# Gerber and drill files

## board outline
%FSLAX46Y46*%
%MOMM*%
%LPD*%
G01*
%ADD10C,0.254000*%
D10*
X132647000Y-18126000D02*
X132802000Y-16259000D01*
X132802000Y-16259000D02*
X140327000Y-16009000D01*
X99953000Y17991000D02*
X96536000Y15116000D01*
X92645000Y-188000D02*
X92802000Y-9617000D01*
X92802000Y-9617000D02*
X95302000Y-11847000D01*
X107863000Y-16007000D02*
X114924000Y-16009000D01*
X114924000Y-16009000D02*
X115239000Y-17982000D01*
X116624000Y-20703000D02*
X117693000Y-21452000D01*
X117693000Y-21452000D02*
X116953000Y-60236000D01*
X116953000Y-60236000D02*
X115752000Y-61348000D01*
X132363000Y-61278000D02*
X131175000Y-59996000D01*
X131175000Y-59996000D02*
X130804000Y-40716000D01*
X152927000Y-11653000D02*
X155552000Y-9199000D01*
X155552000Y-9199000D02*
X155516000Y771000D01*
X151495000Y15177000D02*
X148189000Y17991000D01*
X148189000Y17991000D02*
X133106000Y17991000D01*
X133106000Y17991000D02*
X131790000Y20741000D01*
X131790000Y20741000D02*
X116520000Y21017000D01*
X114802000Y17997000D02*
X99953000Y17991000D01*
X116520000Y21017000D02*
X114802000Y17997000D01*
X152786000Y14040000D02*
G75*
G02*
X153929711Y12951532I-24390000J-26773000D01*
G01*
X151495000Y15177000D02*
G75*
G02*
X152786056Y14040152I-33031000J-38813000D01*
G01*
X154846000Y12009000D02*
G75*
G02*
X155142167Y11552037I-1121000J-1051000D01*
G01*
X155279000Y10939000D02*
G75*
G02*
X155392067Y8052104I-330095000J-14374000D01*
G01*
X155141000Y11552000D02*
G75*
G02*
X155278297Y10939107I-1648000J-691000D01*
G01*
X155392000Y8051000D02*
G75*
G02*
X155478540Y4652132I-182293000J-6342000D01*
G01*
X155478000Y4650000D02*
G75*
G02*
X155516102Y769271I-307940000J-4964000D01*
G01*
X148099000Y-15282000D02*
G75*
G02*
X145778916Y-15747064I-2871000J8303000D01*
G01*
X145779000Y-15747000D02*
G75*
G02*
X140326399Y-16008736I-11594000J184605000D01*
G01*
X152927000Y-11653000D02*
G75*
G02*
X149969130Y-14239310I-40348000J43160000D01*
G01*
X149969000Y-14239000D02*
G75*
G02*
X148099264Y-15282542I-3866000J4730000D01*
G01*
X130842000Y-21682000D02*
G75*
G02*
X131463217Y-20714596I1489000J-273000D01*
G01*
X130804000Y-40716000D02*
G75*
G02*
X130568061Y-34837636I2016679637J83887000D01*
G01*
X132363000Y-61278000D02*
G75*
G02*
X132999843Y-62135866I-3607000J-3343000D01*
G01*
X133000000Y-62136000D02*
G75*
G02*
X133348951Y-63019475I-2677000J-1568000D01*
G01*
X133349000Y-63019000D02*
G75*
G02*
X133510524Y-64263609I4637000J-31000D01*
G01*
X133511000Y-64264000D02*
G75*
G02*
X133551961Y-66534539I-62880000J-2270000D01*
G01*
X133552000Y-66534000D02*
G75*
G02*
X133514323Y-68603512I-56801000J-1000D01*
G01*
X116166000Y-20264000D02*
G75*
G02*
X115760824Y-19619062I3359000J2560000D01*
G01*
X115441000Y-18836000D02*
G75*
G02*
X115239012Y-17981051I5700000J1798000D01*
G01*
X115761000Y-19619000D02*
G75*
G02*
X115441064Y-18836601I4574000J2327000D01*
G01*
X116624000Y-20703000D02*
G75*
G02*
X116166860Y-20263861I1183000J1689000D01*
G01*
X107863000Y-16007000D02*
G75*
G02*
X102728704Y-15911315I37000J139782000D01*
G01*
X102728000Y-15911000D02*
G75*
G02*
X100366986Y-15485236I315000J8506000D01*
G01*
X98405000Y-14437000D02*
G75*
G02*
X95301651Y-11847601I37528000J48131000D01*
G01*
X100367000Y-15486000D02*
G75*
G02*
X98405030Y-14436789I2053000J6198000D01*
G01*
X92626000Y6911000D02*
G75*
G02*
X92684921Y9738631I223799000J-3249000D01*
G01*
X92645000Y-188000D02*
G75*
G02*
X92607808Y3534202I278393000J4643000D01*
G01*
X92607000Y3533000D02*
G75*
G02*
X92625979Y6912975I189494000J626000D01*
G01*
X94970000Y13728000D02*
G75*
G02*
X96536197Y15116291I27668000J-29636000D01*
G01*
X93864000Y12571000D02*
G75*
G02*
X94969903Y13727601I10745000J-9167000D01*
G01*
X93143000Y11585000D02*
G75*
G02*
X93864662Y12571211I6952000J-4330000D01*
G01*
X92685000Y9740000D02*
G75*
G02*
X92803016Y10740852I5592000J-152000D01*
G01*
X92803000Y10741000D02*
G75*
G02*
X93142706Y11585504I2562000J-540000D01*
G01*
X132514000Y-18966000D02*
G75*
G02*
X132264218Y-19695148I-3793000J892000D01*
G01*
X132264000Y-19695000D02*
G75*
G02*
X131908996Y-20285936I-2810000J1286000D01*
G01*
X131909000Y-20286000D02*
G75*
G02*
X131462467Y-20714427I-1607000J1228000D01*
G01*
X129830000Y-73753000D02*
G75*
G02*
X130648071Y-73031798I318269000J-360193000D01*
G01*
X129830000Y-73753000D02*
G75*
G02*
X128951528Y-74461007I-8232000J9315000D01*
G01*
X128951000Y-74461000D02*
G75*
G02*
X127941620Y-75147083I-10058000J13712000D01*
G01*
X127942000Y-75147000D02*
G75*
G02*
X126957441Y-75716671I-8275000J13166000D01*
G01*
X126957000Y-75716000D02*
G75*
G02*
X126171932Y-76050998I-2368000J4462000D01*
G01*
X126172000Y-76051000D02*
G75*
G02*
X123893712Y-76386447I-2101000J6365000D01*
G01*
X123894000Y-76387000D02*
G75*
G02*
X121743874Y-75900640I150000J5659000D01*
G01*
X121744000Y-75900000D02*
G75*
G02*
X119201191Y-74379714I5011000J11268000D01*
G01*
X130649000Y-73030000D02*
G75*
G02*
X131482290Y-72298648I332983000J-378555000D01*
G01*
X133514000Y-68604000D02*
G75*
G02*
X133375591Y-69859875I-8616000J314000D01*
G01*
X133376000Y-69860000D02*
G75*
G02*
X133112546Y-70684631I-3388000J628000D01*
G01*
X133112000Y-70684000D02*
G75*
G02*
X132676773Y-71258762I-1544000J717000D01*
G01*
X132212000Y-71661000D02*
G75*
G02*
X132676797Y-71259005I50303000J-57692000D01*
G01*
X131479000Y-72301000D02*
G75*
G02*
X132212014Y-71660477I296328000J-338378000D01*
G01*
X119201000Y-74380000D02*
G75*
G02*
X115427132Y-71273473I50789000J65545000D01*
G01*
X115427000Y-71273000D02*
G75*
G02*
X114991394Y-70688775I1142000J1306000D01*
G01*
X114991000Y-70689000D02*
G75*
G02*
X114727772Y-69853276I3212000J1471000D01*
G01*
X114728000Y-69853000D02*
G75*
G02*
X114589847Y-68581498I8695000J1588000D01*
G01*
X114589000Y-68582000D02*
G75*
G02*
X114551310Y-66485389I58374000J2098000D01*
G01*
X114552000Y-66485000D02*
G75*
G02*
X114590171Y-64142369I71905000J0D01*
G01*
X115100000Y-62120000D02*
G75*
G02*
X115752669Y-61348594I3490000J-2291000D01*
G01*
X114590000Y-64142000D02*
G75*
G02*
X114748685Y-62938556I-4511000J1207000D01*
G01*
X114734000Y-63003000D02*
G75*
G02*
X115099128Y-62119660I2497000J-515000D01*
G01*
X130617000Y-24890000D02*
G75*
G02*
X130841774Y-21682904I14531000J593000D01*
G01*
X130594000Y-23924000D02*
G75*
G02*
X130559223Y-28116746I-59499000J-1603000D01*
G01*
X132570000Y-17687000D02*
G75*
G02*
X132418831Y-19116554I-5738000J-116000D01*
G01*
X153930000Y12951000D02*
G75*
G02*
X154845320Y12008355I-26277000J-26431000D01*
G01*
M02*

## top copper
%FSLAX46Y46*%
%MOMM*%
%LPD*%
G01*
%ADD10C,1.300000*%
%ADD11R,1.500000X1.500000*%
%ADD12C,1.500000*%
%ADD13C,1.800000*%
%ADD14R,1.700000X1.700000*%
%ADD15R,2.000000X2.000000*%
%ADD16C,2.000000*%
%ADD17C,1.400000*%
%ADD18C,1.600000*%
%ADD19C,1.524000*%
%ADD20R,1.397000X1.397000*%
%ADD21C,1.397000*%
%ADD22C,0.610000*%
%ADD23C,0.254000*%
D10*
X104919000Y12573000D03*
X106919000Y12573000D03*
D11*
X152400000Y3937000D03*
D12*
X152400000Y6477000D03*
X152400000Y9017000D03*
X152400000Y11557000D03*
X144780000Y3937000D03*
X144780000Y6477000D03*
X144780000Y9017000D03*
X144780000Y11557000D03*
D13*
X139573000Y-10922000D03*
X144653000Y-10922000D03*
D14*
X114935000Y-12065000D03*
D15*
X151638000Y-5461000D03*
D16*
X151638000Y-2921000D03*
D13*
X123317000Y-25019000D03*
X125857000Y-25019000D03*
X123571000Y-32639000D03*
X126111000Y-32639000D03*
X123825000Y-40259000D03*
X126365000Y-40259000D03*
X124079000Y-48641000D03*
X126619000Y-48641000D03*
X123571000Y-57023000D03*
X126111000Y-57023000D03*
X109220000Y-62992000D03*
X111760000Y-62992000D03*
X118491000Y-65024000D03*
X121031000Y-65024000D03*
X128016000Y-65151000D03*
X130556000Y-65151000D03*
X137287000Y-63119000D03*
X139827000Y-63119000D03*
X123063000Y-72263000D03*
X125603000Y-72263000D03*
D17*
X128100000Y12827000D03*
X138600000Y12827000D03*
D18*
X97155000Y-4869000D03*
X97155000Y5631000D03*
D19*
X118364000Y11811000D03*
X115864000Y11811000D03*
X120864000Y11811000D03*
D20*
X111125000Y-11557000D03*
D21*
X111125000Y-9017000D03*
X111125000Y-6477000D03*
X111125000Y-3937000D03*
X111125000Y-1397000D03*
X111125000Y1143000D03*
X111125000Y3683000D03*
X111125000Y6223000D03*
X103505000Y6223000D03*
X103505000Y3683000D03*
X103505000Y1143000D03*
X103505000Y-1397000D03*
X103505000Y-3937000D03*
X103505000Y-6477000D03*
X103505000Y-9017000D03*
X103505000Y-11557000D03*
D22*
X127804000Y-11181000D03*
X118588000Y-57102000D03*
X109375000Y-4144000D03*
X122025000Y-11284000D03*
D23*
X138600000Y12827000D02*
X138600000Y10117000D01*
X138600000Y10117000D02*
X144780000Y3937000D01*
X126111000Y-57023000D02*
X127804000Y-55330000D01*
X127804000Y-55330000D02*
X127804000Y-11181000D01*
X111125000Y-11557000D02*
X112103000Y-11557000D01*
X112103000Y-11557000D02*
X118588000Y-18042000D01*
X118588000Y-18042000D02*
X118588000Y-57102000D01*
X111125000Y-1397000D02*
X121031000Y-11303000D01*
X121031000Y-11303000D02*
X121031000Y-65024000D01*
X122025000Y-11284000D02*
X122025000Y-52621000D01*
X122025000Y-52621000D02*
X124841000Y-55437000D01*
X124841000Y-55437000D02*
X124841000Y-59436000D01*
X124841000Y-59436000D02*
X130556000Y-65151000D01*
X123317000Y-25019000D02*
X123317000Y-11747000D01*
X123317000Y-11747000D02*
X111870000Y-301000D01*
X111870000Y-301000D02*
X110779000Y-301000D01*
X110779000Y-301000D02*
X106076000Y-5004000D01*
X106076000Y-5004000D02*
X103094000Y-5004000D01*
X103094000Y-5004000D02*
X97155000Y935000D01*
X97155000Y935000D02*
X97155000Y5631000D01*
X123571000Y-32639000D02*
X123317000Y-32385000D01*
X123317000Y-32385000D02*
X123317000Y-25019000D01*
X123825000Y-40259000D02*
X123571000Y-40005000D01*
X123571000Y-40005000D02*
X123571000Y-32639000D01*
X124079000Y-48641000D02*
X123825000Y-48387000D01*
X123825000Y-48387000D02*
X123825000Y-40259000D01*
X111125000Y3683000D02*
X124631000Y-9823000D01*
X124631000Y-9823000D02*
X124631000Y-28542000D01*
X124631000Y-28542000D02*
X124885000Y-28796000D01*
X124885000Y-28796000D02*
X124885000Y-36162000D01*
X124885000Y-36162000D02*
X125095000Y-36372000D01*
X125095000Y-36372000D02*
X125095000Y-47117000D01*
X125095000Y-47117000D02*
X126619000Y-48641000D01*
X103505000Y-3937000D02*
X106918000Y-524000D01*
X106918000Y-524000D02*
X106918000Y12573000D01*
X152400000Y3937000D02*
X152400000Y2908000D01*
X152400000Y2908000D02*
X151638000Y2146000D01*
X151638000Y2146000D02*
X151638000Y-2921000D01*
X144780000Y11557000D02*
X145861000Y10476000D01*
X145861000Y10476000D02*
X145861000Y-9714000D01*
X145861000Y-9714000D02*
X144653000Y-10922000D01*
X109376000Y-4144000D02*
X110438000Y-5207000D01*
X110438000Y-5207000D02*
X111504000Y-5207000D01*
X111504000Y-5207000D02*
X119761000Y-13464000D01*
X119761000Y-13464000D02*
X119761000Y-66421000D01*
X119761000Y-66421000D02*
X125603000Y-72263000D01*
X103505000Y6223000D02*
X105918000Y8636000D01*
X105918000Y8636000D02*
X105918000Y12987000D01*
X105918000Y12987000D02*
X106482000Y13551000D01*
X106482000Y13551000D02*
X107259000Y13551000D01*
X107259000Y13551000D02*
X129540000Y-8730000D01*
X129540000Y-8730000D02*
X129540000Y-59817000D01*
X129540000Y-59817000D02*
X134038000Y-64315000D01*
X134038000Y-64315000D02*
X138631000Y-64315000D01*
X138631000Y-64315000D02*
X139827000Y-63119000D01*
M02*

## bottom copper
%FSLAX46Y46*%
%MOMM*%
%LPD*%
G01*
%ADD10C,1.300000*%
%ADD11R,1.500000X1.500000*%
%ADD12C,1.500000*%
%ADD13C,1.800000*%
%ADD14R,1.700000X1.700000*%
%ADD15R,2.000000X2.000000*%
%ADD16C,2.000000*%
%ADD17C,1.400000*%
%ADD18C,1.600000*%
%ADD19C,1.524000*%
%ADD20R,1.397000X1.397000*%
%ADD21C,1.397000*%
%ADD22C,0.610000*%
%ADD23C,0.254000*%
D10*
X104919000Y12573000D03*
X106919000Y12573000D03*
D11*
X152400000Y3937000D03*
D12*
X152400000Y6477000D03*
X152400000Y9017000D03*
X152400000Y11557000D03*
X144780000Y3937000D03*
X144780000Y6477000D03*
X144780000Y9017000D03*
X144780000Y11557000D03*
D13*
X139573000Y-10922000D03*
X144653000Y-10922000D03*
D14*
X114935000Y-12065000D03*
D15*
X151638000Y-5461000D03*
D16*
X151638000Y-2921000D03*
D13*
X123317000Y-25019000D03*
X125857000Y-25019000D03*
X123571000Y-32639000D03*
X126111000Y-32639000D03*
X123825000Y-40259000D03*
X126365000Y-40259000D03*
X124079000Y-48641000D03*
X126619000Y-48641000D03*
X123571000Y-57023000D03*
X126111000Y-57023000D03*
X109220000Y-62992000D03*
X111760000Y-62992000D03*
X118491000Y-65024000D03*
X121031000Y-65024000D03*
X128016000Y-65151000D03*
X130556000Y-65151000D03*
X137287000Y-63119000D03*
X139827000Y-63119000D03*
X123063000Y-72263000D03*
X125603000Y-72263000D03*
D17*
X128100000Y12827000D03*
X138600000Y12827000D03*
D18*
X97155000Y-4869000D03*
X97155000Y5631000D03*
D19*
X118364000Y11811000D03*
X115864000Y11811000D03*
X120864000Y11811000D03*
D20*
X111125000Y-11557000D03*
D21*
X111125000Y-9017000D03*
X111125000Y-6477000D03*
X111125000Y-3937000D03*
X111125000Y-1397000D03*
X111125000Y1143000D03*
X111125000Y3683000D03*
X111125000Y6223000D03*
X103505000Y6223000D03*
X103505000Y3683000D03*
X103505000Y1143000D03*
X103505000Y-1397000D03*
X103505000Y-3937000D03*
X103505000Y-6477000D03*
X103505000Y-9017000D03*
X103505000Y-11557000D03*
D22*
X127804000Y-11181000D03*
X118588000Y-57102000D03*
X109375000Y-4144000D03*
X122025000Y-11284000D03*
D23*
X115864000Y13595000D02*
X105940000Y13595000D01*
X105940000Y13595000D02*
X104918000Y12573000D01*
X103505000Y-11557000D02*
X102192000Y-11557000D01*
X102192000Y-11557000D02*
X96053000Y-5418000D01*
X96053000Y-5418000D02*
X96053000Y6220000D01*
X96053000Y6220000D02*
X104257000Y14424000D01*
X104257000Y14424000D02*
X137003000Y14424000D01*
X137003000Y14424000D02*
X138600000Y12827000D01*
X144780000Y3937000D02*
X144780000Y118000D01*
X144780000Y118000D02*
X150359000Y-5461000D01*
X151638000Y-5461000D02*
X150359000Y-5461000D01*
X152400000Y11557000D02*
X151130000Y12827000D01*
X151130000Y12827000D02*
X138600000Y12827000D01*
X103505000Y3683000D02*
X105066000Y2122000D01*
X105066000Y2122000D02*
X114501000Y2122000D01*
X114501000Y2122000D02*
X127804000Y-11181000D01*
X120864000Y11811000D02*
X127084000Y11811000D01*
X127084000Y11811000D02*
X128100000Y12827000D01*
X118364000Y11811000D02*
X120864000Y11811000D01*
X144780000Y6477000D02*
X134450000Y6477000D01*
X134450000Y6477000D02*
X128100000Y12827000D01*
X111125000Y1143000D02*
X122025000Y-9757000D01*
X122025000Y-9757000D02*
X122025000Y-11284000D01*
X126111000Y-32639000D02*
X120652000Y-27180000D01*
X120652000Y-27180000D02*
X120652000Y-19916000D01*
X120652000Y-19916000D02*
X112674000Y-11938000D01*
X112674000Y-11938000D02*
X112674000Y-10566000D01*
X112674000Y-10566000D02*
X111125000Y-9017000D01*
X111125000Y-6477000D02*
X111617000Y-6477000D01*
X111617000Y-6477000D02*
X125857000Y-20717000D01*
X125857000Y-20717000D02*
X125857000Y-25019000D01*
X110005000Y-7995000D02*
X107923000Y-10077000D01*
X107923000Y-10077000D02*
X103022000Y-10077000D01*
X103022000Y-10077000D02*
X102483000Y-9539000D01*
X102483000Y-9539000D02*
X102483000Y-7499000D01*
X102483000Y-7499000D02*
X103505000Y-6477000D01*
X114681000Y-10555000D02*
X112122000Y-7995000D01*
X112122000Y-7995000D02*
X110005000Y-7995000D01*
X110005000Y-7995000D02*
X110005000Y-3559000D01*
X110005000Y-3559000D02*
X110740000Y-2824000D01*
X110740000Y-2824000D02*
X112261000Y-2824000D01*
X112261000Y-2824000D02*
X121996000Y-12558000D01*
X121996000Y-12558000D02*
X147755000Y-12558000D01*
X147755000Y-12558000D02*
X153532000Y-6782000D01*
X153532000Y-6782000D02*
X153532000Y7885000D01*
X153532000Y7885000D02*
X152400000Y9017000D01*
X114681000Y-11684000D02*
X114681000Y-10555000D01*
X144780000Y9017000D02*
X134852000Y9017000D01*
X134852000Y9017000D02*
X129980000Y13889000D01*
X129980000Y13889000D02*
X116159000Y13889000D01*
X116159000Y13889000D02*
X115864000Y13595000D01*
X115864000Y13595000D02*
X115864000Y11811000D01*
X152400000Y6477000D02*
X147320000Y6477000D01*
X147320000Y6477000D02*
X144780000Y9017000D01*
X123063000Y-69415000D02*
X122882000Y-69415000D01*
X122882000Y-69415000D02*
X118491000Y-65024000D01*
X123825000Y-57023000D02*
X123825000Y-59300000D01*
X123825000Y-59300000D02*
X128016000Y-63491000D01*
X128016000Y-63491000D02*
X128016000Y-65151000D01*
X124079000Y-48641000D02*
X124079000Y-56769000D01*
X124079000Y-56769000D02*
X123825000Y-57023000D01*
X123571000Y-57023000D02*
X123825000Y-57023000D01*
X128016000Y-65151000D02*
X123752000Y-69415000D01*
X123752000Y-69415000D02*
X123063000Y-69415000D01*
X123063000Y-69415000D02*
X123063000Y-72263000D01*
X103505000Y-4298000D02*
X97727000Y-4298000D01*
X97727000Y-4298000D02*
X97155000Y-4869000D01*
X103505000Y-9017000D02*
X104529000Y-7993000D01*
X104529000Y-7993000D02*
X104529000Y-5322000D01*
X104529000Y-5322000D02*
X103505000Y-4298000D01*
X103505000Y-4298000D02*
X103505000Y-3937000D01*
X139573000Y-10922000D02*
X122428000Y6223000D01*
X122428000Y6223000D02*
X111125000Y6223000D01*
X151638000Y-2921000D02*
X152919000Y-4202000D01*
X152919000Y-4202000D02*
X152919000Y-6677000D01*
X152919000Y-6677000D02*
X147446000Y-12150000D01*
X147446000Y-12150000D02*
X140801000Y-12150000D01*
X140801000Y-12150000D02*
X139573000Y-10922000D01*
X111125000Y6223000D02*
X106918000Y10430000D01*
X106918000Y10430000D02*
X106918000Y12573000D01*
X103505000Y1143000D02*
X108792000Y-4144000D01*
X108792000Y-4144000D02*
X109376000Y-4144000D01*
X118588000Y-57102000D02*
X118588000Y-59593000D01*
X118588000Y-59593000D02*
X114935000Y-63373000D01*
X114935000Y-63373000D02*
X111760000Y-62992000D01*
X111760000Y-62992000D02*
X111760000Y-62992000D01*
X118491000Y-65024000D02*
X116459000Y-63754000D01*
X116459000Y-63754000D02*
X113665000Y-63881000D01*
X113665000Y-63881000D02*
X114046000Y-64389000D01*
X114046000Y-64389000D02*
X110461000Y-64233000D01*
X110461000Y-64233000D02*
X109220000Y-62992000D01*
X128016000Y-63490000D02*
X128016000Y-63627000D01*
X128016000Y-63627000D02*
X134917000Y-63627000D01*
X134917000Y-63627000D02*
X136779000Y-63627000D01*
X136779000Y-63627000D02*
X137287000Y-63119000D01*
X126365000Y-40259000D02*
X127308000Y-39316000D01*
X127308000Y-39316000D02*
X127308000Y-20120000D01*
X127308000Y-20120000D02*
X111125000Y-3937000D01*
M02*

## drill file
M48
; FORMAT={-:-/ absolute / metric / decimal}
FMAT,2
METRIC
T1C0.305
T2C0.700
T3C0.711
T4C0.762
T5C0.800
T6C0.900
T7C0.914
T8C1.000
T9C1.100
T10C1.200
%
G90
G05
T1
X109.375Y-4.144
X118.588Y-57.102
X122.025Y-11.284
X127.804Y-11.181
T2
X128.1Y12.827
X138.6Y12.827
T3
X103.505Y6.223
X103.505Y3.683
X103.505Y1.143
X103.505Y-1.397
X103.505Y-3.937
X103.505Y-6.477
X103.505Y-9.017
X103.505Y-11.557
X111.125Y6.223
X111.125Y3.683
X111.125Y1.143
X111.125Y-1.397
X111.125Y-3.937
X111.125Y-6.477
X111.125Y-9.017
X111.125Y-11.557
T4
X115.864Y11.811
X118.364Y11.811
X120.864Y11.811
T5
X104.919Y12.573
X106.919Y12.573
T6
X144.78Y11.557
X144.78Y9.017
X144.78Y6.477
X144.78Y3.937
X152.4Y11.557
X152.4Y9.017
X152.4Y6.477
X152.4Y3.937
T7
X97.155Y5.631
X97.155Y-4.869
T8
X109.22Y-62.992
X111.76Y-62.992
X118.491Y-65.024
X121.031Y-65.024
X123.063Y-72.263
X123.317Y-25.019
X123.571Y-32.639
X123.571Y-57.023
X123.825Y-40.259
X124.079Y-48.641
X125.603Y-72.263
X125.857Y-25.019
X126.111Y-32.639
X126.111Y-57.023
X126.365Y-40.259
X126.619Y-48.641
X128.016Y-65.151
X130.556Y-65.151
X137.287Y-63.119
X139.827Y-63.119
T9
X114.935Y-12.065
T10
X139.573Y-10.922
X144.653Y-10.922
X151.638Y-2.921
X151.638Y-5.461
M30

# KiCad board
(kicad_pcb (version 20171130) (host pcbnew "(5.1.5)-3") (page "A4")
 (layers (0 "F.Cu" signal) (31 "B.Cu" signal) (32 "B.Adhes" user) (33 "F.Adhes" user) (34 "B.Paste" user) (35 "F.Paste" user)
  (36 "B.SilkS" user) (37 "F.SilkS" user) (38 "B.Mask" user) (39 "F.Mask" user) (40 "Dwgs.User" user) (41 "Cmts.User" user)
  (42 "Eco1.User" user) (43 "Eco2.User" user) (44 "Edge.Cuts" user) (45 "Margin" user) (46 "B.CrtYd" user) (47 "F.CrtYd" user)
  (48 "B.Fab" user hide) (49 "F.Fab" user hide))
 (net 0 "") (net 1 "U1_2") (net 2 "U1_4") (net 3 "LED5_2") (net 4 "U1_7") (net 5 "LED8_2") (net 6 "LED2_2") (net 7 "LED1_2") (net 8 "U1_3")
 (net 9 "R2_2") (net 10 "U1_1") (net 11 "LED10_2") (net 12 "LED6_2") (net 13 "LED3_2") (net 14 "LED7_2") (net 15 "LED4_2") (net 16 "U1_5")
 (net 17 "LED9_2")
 (segment (start 115.864 -13.595) (end 105.94 -13.595) (width 0.254) (layer "B.Cu") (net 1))
 (segment (start 105.94 -13.595) (end 104.918 -12.573) (width 0.254) (layer "B.Cu") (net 1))
 (segment (start 103.505 11.557) (end 102.192 11.557) (width 0.254) (layer "B.Cu") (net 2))
 (segment (start 102.192 11.557) (end 96.053 5.418) (width 0.254) (layer "B.Cu") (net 2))
 (segment (start 96.053 5.418) (end 96.053 -6.22) (width 0.254) (layer "B.Cu") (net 2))
 (segment (start 96.053 -6.22) (end 104.257 -14.424) (width 0.254) (layer "B.Cu") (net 2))
 (segment (start 104.257 -14.424) (end 137.003 -14.424) (width 0.254) (layer "B.Cu") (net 2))
 (segment (start 137.003 -14.424) (end 138.6 -12.827) (width 0.254) (layer "B.Cu") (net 2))
 (segment (start 144.78 -3.937) (end 144.78 -0.118) (width 0.254) (layer "B.Cu") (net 2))
 (segment (start 144.78 -0.118) (end 150.359 5.461) (width 0.254) (layer "B.Cu") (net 2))
 (segment (start 151.638 5.461) (end 150.359 5.461) (width 0.254) (layer "B.Cu") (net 2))
 (segment (start 152.4 -11.557) (end 151.13 -12.827) (width 0.254) (layer "B.Cu") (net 2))
 (segment (start 151.13 -12.827) (end 138.6 -12.827) (width 0.254) (layer "B.Cu") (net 2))
 (segment (start 103.505 -3.683) (end 105.066 -2.122) (width 0.254) (layer "B.Cu") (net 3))
 (segment (start 105.066 -2.122) (end 114.501 -2.122) (width 0.254) (layer "B.Cu") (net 3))
 (segment (start 114.501 -2.122) (end 127.804 11.181) (width 0.254) (layer "B.Cu") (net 3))
 (segment (start 120.864 -11.811) (end 127.084 -11.811) (width 0.254) (layer "B.Cu") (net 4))
 (segment (start 127.084 -11.811) (end 128.1 -12.827) (width 0.254) (layer "B.Cu") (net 4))
 (segment (start 118.364 -11.811) (end 120.864 -11.811) (width 0.254) (layer "B.Cu") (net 4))
 (segment (start 144.78 -6.477) (end 134.45 -6.477) (width 0.254) (layer "B.Cu") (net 4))
 (segment (start 134.45 -6.477) (end 128.1 -12.827) (width 0.254) (layer "B.Cu") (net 4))
 (segment (start 111.125 -1.143) (end 122.025 9.757) (width 0.254) (layer "B.Cu") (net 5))
 (segment (start 122.025 9.757) (end 122.025 11.284) (width 0.254) (layer "B.Cu") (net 5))
 (segment (start 126.111 32.639) (end 120.652 27.18) (width 0.254) (layer "B.Cu") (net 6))
 (segment (start 120.652 27.18) (end 120.652 19.916) (width 0.254) (layer "B.Cu") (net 6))
 (segment (start 120.652 19.916) (end 112.674 11.938) (width 0.254) (layer "B.Cu") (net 6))
 (segment (start 112.674 11.938) (end 112.674 10.566) (width 0.254) (layer "B.Cu") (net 6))
 (segment (start 112.674 10.566) (end 111.125 9.017) (width 0.254) (layer "B.Cu") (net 6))
 (segment (start 111.125 6.477) (end 111.617 6.477) (width 0.254) (layer "B.Cu") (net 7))
 (segment (start 111.617 6.477) (end 125.857 20.717) (width 0.254) (layer "B.Cu") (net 7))
 (segment (start 125.857 20.717) (end 125.857 25.019) (width 0.254) (layer "B.Cu") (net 7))
 (segment (start 110.005 7.995) (end 107.923 10.077) (width 0.254) (layer "B.Cu") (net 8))
 (segment (start 107.923 10.077) (end 103.022 10.077) (width 0.254) (layer "B.Cu") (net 8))
 (segment (start 103.022 10.077) (end 102.483 9.539) (width 0.254) (layer "B.Cu") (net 8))
 (segment (start 102.483 9.539) (end 102.483 7.499) (width 0.254) (layer "B.Cu") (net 8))
 (segment (start 102.483 7.499) (end 103.505 6.477) (width 0.254) (layer "B.Cu") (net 8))
 (segment (start 114.681 10.555) (end 112.122 7.995) (width 0.254) (layer "B.Cu") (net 8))
 (segment (start 112.122 7.995) (end 110.005 7.995) (width 0.254) (layer "B.Cu") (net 8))
 (segment (start 110.005 7.995) (end 110.005 3.559) (width 0.254) (layer "B.Cu") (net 8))
 (segment (start 110.005 3.559) (end 110.74 2.824) (width 0.254) (layer "B.Cu") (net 8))
 (segment (start 110.74 2.824) (end 112.261 2.824) (width 0.254) (layer "B.Cu") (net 8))
 (segment (start 112.261 2.824) (end 121.996 12.558) (width 0.254) (layer "B.Cu") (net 8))
 (segment (start 121.996 12.558) (end 147.755 12.558) (width 0.254) (layer "B.Cu") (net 8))
 (segment (start 147.755 12.558) (end 153.532 6.782) (width 0.254) (layer "B.Cu") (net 8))
 (segment (start 153.532 6.782) (end 153.532 -7.885) (width 0.254) (layer "B.Cu") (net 8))
 (segment (start 153.532 -7.885) (end 152.4 -9.017) (width 0.254) (layer "B.Cu") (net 8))
 (segment (start 114.681 11.684) (end 114.681 10.555) (width 0.254) (layer "B.Cu") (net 8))
 (segment (start 144.78 -9.017) (end 134.852 -9.017) (width 0.254) (layer "B.Cu") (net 1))
 (segment (start 134.852 -9.017) (end 129.98 -13.889) (width 0.254) (layer "B.Cu") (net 1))
 (segment (start 129.98 -13.889) (end 116.159 -13.889) (width 0.254) (layer "B.Cu") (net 1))
 (segment (start 116.159 -13.889) (end 115.864 -13.595) (width 0.254) (layer "B.Cu") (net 1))
 (segment (start 115.864 -13.595) (end 115.864 -11.811) (width 0.254) (layer "B.Cu") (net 1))
 (segment (start 152.4 -6.477) (end 147.32 -6.477) (width 0.254) (layer "B.Cu") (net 1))
 (segment (start 147.32 -6.477) (end 144.78 -9.017) (width 0.254) (layer "B.Cu") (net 1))
 (segment (start 123.063 69.415) (end 122.882 69.415) (width 0.254) (layer "B.Cu") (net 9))
 (segment (start 122.882 69.415) (end 118.491 65.024) (width 0.254) (layer "B.Cu") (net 9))
 (segment (start 123.825 57.023) (end 123.825 59.3) (width 0.254) (layer "B.Cu") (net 9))
 (segment (start 123.825 59.3) (end 128.016 63.491) (width 0.254) (layer "B.Cu") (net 9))
 (segment (start 128.016 63.491) (end 128.016 65.151) (width 0.254) (layer "B.Cu") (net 9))
 (segment (start 124.079 48.641) (end 124.079 56.769) (width 0.254) (layer "B.Cu") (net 9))
 (segment (start 124.079 56.769) (end 123.825 57.023) (width 0.254) (layer "B.Cu") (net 9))
 (segment (start 123.571 57.023) (end 123.825 57.023) (width 0.254) (layer "B.Cu") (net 9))
 (segment (start 128.016 65.151) (end 123.752 69.415) (width 0.254) (layer "B.Cu") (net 9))
 (segment (start 123.752 69.415) (end 123.063 69.415) (width 0.254) (layer "B.Cu") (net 9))
 (segment (start 123.063 69.415) (end 123.063 72.263) (width 0.254) (layer "B.Cu") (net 9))
 (segment (start 103.505 4.298) (end 97.727 4.298) (width 0.254) (layer "B.Cu") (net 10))
 (segment (start 97.727 4.298) (end 97.155 4.869) (width 0.254) (layer "B.Cu") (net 10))
 (segment (start 103.505 9.017) (end 104.529 7.993) (width 0.254) (layer "B.Cu") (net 10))
 (segment (start 104.529 7.993) (end 104.529 5.322) (width 0.254) (layer "B.Cu") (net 10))
 (segment (start 104.529 5.322) (end 103.505 4.298) (width 0.254) (layer "B.Cu") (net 10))
 (segment (start 103.505 4.298) (end 103.505 3.937) (width 0.254) (layer "B.Cu") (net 10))
 (segment (start 139.573 10.922) (end 122.428 -6.223) (width 0.254) (layer "B.Cu") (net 10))
 (segment (start 122.428 -6.223) (end 111.125 -6.223) (width 0.254) (layer "B.Cu") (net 10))
 (segment (start 151.638 2.921) (end 152.919 4.202) (width 0.254) (layer "B.Cu") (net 10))
 (segment (start 152.919 4.202) (end 152.919 6.677) (width 0.254) (layer "B.Cu") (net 10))
 (segment (start 152.919 6.677) (end 147.446 12.15) (width 0.254) (layer "B.Cu") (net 10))
 (segment (start 147.446 12.15) (end 140.801 12.15) (width 0.254) (layer "B.Cu") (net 10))
 (segment (start 140.801 12.15) (end 139.573 10.922) (width 0.254) (layer "B.Cu") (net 10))
 (segment (start 111.125 -6.223) (end 106.918 -10.43) (width 0.254) (layer "B.Cu") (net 10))
 (segment (start 106.918 -10.43) (end 106.918 -12.573) (width 0.254) (layer "B.Cu") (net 10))
 (segment (start 103.505 -1.143) (end 108.792 4.144) (width 0.254) (layer "B.Cu") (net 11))
 (segment (start 108.792 4.144) (end 109.376 4.144) (width 0.254) (layer "B.Cu") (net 11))
 (segment (start 118.588 57.102) (end 118.588 59.593) (width 0.254) (layer "B.Cu") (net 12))
 (segment (start 118.588 59.593) (end 114.935 63.373) (width 0.254) (layer "B.Cu") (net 12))
 (segment (start 114.935 63.373) (end 111.76 62.992) (width 0.254) (layer "B.Cu") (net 12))
 (segment (start 111.76 62.992) (end 111.76 62.992) (width 0.254) (layer "B.Cu") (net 12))
 (segment (start 118.491 65.024) (end 116.459 63.754) (width 0.254) (layer "B.Cu") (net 9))
 (segment (start 116.459 63.754) (end 113.665 63.881) (width 0.254) (layer "B.Cu") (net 9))
 (segment (start 113.665 63.881) (end 114.046 64.389) (width 0.254) (layer "B.Cu") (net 9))
 (segment (start 114.046 64.389) (end 110.461 64.233) (width 0.254) (layer "B.Cu") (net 9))
 (segment (start 110.461 64.233) (end 109.22 62.992) (width 0.254) (layer "B.Cu") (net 9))
 (segment (start 128.016 63.49) (end 128.016 63.627) (width 0.254) (layer "B.Cu") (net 9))
 (segment (start 128.016 63.627) (end 134.917 63.627) (width 0.254) (layer "B.Cu") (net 9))
 (segment (start 134.917 63.627) (end 136.779 63.627) (width 0.254) (layer "B.Cu") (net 9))
 (segment (start 136.779 63.627) (end 137.287 63.119) (width 0.254) (layer "B.Cu") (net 9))
 (segment (start 126.365 40.259) (end 127.308 39.316) (width 0.254) (layer "B.Cu") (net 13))
 (segment (start 127.308 39.316) (end 127.308 20.12) (width 0.254) (layer "B.Cu") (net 13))
 (segment (start 127.308 20.12) (end 111.125 3.937) (width 0.254) (layer "B.Cu") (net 13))
 (gr_line (start 132.647 18.126) (end 132.802 16.259) (width 0.254) (layer "Edge.Cuts"))
 (gr_line (start 132.802 16.259) (end 140.327 16.009) (width 0.254) (layer "Edge.Cuts"))
 (gr_line (start 99.953 -17.991) (end 96.536 -15.116) (width 0.254) (layer "Edge.Cuts"))
 (gr_line (start 92.645 0.188) (end 92.802 9.617) (width 0.254) (layer "Edge.Cuts"))
 (gr_line (start 92.802 9.617) (end 95.302 11.847) (width 0.254) (layer "Edge.Cuts"))
 (gr_line (start 107.863 16.007) (end 114.924 16.009) (width 0.254) (layer "Edge.Cuts"))
 (gr_line (start 114.924 16.009) (end 115.239 17.982) (width 0.254) (layer "Edge.Cuts"))
 (gr_line (start 116.624 20.703) (end 117.693 21.452) (width 0.254) (layer "Edge.Cuts"))
 (gr_line (start 117.693 21.452) (end 116.953 60.236) (width 0.254) (layer "Edge.Cuts"))
 (gr_line (start 116.953 60.236) (end 115.752 61.348) (width 0.254) (layer "Edge.Cuts"))
 (gr_line (start 132.363 61.278) (end 131.175 59.996) (width 0.254) (layer "Edge.Cuts"))
 (gr_line (start 131.175 59.996) (end 130.804 40.716) (width 0.254) (layer "Edge.Cuts"))
 (gr_line (start 152.927 11.653) (end 155.552 9.199) (width 0.254) (layer "Edge.Cuts"))
 (gr_line (start 155.552 9.199) (end 155.516 -0.771) (width 0.254) (layer "Edge.Cuts"))
 (gr_line (start 151.495 -15.177) (end 148.189 -17.991) (width 0.254) (layer "Edge.Cuts"))
 (gr_line (start 148.189 -17.991) (end 133.106 -17.991) (width 0.254) (layer "Edge.Cuts"))
 (gr_line (start 133.106 -17.991) (end 131.79 -20.741) (width 0.254) (layer "Edge.Cuts"))
 (gr_line (start 131.79 -20.741) (end 116.52 -21.017) (width 0.254) (layer "Edge.Cuts"))
 (gr_line (start 114.802 -17.997) (end 99.953 -17.991) (width 0.254) (layer "Edge.Cuts"))
 (gr_line (start 116.52 -21.017) (end 114.802 -17.997) (width 0.254) (layer "Edge.Cuts"))
 (gr_arc (start 128.396 12.733) (end 152.786 -14.04) (angle 2.498) (width 0.254) (layer "Edge.Cuts"))
 (gr_arc (start 118.464 23.636) (end 151.495 -15.177) (angle 1.934) (width 0.254) (layer "Edge.Cuts"))
 (gr_arc (start 153.725 -10.958) (end 154.846 -12.009) (angle 20.412) (width 0.254) (layer "Edge.Cuts"))
 (gr_arc (start -174.816 3.435) (end 155.279 -10.939) (angle 0.501) (width 0.254) (layer "Edge.Cuts"))
 (gr_arc (start 153.493 -10.861) (end 155.141 -11.552) (angle 20.243) (width 0.254) (layer "Edge.Cuts"))
 (gr_arc (start -26.901 -1.709) (end 155.392 -8.051) (angle 1.068) (width 0.254) (layer "Edge.Cuts"))
 (gr_arc (start -152.462 0.314) (end 155.478 -4.65) (angle 0.722) (width 0.254) (layer "Edge.Cuts"))
 (gr_arc (start 145.228 6.979) (end 148.099 15.282) (angle 15.479) (width 0.254) (layer "Edge.Cuts"))
 (gr_arc (start 134.185 -168.858) (end 145.779 15.747) (angle 1.691) (width 0.254) (layer "Edge.Cuts"))
 (gr_arc (start 112.579 -31.507) (end 152.927 11.653) (angle 3.811) (width 0.254) (layer "Edge.Cuts"))
 (gr_arc (start 146.103 9.509) (end 149.969 14.239) (angle 20.187) (width 0.254) (layer "Edge.Cuts"))
 (gr_arc (start 132.331 21.955) (end 130.842 21.682) (angle 44.634) (width 0.254) (layer "Edge.Cuts"))
 (gr_arc (start 4493.463 -43.171) (end 130.804 40.716) (angle 0.167) (width 0.254) (layer "Edge.Cuts"))
 (gr_arc (start 128.756 64.621) (end 132.363 61.278) (angle 12.472) (width 0.254) (layer "Edge.Cuts"))
 (gr_arc (start 130.323 63.704) (end 133 62.136) (angle 17.612) (width 0.254) (layer "Edge.Cuts"))
 (gr_arc (start 137.986 63.05) (end 133.349 63.019) (angle 344.445) (width 0.254) (layer "Edge.Cuts"))
 (gr_arc (start 70.631 66.534) (end 133.511 64.264) (angle 2.068) (width 0.254) (layer "Edge.Cuts"))
 (gr_arc (start 76.751 66.535) (end 133.552 66.534) (angle 2.088) (width 0.254) (layer "Edge.Cuts"))
 (gr_arc (start 119.525 17.704) (end 116.166 20.264) (angle 10.347) (width 0.254) (layer "Edge.Cuts"))
 (gr_arc (start 121.141 17.038) (end 115.441 18.836) (angle 8.429) (width 0.254) (layer "Edge.Cuts"))
 (gr_arc (start 120.335 17.292) (end 115.761 19.619) (angle 9.448) (width 0.254) (layer "Edge.Cuts"))
 (gr_arc (start 117.807 19.014) (end 116.624 20.703) (angle 17.683) (width 0.254) (layer "Edge.Cuts"))
 (gr_arc (start 107.9 -123.775) (end 107.863 16.007) (angle 2.105) (width 0.254) (layer "Edge.Cuts"))
 (gr_arc (start 103.043 7.405) (end 102.728 15.911) (angle 16.203) (width 0.254) (layer "Edge.Cuts"))
 (gr_arc (start 135.933 -33.694) (end 98.405 14.437) (angle 3.795) (width 0.254) (layer "Edge.Cuts"))
 (gr_arc (start 102.42 9.288) (end 100.367 15.486) (angle 19.62) (width 0.254) (layer "Edge.Cuts"))
 (gr_arc (start 316.425 -3.662) (end 92.626 -6.911) (angle 0.724) (width 0.254) (layer "Edge.Cuts"))
 (gr_arc (start 371.038 -4.455) (end 92.645 0.188) (angle 0.766) (width 0.254) (layer "Edge.Cuts"))
 (gr_arc (start 282.101 -4.159) (end 92.607 -3.533) (angle 1.022) (width 0.254) (layer "Edge.Cuts"))
 (gr_arc (start 122.638 15.908) (end 94.97 -13.728) (angle 2.958) (width 0.254) (layer "Edge.Cuts"))
 (gr_arc (start 104.609 -3.404) (end 93.864 -12.571) (angle 6.495) (width 0.254) (layer "Edge.Cuts"))
 (gr_arc (start 100.095 -7.255) (end 93.143 -11.585) (angle 8.557) (width 0.254) (layer "Edge.Cuts"))
 (gr_arc (start 98.277 -9.588) (end 92.685 -9.74) (angle 10.336) (width 0.254) (layer "Edge.Cuts"))
 (gr_arc (start 95.365 -10.201) (end 92.803 -10.741) (angle 20.021) (width 0.254) (layer "Edge.Cuts"))
 (gr_arc (start 128.721 18.074) (end 132.514 18.966) (angle 11.352) (width 0.254) (layer "Edge.Cuts"))
 (gr_arc (start 129.454 18.409) (end 132.264 19.695) (angle 12.808) (width 0.254) (layer "Edge.Cuts"))
 (gr_arc (start 130.302 19.058) (end 131.909 20.286) (angle 17.6) (width 0.254) (layer "Edge.Cuts"))
 (gr_arc (start 448.099 433.946) (end 129.83 73.753) (angle 0.13) (width 0.254) (layer "Edge.Cuts"))
 (gr_arc (start 121.598 64.438) (end 129.83 73.753) (angle 5.202) (width 0.254) (layer "Edge.Cuts"))
 (gr_arc (start 118.893 60.749) (end 128.951 74.461) (angle 4.113) (width 0.254) (layer "Edge.Cuts"))
 (gr_arc (start 119.667 61.981) (end 127.942 75.147) (angle 4.192) (width 0.254) (layer "Edge.Cuts"))
 (gr_arc (start 124.589 71.254) (end 126.957 75.716) (angle 9.693) (width 0.254) (layer "Edge.Cuts"))
 (gr_arc (start 124.071 69.686) (end 126.172 76.051) (angle 19.783) (width 0.254) (layer "Edge.Cuts"))
 (gr_arc (start 124.044 70.728) (end 123.894 76.387) (angle 22.455) (width 0.254) (layer "Edge.Cuts"))
 (gr_arc (start 126.755 64.632) (end 121.744 75.9) (angle 13.798) (width 0.254) (layer "Edge.Cuts"))
 (gr_arc (start 463.632 451.585) (end 130.649 73.03) (angle 0.126) (width 0.254) (layer "Edge.Cuts"))
 (gr_arc (start 124.898 68.29) (end 133.514 68.604) (angle 8.404) (width 0.254) (layer "Edge.Cuts"))
 (gr_arc (start 129.988 69.232) (end 133.376 69.86) (angle 14.433) (width 0.254) (layer "Edge.Cuts"))
 (gr_arc (start 131.568 69.967) (end 133.112 70.684) (angle 24.45) (width 0.254) (layer "Edge.Cuts"))
 (gr_arc (start 182.515 129.353) (end 132.212 71.661) (angle 0.46) (width 0.254) (layer "Edge.Cuts"))
 (gr_arc (start 427.807 410.679) (end 131.479 72.301) (angle 0.124) (width 0.254) (layer "Edge.Cuts"))
 (gr_arc (start 169.99 8.835) (end 119.201 74.38) (angle 3.378) (width 0.254) (layer "Edge.Cuts"))
 (gr_arc (start 116.569 69.967) (end 115.427 71.273) (angle 24.248) (width 0.254) (layer "Edge.Cuts"))
 (gr_arc (start 118.203 69.218) (end 114.991 70.689) (angle 14.247) (width 0.254) (layer "Edge.Cuts"))
 (gr_arc (start 123.423 68.265) (end 114.728 69.853) (angle 8.298) (width 0.254) (layer "Edge.Cuts"))
 (gr_arc (start 172.963 66.484) (end 114.589 68.582) (angle 2.057) (width 0.254) (layer "Edge.Cuts"))
 (gr_arc (start 186.457 66.485) (end 114.552 66.485) (angle 1.867) (width 0.254) (layer "Edge.Cuts"))
 (gr_arc (start 118.59 64.411) (end 115.1 62.12) (angle 13.902) (width 0.254) (layer "Edge.Cuts"))
 (gr_arc (start 110.079 62.935) (end 114.59 64.142) (angle 345.064) (width 0.254) (layer "Edge.Cuts"))
 (gr_arc (start 117.231 63.518) (end 114.734 63.003) (angle 21.608) (width 0.254) (layer "Edge.Cuts"))
 (gr_arc (start 145.148 24.297) (end 130.617 24.89) (angle 12.692) (width 0.254) (layer "Edge.Cuts"))
 (gr_arc (start 71.095 25.527) (end 130.594 23.924) (angle 4.037) (width 0.254) (layer "Edge.Cuts"))
 (gr_arc (start 126.832 17.803) (end 132.57 17.687) (angle 14.389) (width 0.254) (layer "Edge.Cuts"))
 (gr_arc (start 127.653 13.48) (end 153.93 -12.951) (angle 2.02) (width 0.254) (layer "Edge.Cuts"))
 (segment (start 138.6 -12.827) (end 138.6 -10.117) (width 0.254) (layer "F.Cu") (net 2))
 (segment (start 138.6 -10.117) (end 144.78 -3.937) (width 0.254) (layer "F.Cu") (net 2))
 (segment (start 126.111 57.023) (end 127.804 55.33) (width 0.254) (layer "F.Cu") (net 3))
 (segment (start 127.804 55.33) (end 127.804 11.181) (width 0.254) (layer "F.Cu") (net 3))
 (segment (start 111.125 11.557) (end 112.103 11.557) (width 0.254) (layer "F.Cu") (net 12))
 (segment (start 112.103 11.557) (end 118.588 18.042) (width 0.254) (layer "F.Cu") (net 12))
 (segment (start 118.588 18.042) (end 118.588 57.102) (width 0.254) (layer "F.Cu") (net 12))
 (segment (start 111.125 1.397) (end 121.031 11.303) (width 0.254) (layer "F.Cu") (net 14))
 (segment (start 121.031 11.303) (end 121.031 65.024) (width 0.254) (layer "F.Cu") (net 14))
 (segment (start 122.025 11.284) (end 122.025 52.621) (width 0.254) (layer "F.Cu") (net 5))
 (segment (start 122.025 52.621) (end 124.841 55.437) (width 0.254) (layer "F.Cu") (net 5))
 (segment (start 124.841 55.437) (end 124.841 59.436) (width 0.254) (layer "F.Cu") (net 5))
 (segment (start 124.841 59.436) (end 130.556 65.151) (width 0.254) (layer "F.Cu") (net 5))
 (segment (start 123.317 25.019) (end 123.317 11.747) (width 0.254) (layer "F.Cu") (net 9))
 (segment (start 123.317 11.747) (end 111.87 0.301) (width 0.254) (layer "F.Cu") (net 9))
 (segment (start 111.87 0.301) (end 110.779 0.301) (width 0.254) (layer "F.Cu") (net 9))
 (segment (start 110.779 0.301) (end 106.076 5.004) (width 0.254) (layer "F.Cu") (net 9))
 (segment (start 106.076 5.004) (end 103.094 5.004) (width 0.254) (layer "F.Cu") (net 9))
 (segment (start 103.094 5.004) (end 97.155 -0.935) (width 0.254) (layer "F.Cu") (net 9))
 (segment (start 97.155 -0.935) (end 97.155 -5.631) (width 0.254) (layer "F.Cu") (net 9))
 (segment (start 123.571 32.639) (end 123.317 32.385) (width 0.254) (layer "F.Cu") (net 9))
 (segment (start 123.317 32.385) (end 123.317 25.019) (width 0.254) (layer "F.Cu") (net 9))
 (segment (start 123.825 40.259) (end 123.571 40.005) (width 0.254) (layer "F.Cu") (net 9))
 (segment (start 123.571 40.005) (end 123.571 32.639) (width 0.254) (layer "F.Cu") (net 9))
 (segment (start 124.079 48.641) (end 123.825 48.387) (width 0.254) (layer "F.Cu") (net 9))
 (segment (start 123.825 48.387) (end 123.825 40.259) (width 0.254) (layer "F.Cu") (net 9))
 (segment (start 111.125 -3.683) (end 124.631 9.823) (width 0.254) (layer "F.Cu") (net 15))
 (segment (start 124.631 9.823) (end 124.631 28.542) (width 0.254) (layer "F.Cu") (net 15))
 (segment (start 124.631 28.542) (end 124.885 28.796) (width 0.254) (layer "F.Cu") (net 15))
 (segment (start 124.885 28.796) (end 124.885 36.162) (width 0.254) (layer "F.Cu") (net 15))
 (segment (start 124.885 36.162) (end 125.095 36.372) (width 0.254) (layer "F.Cu") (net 15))
 (segment (start 125.095 36.372) (end 125.095 47.117) (width 0.254) (layer "F.Cu") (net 15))
 (segment (start 125.095 47.117) (end 126.619 48.641) (width 0.254) (layer "F.Cu") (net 15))
 (segment (start 103.505 3.937) (end 106.918 0.524) (width 0.254) (layer "F.Cu") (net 10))
 (segment (start 106.918 0.524) (end 106.918 -12.573) (width 0.254) (layer "F.Cu") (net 10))
 (segment (start 152.4 -3.937) (end 152.4 -2.908) (width 0.254) (layer "F.Cu") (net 10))
 (segment (start 152.4 -2.908) (end 151.638 -2.146) (width 0.254) (layer "F.Cu") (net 10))
 (segment (start 151.638 -2.146) (end 151.638 2.921) (width 0.254) (layer "F.Cu") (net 10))
 (segment (start 144.78 -11.557) (end 145.861 -10.476) (width 0.254) (layer "F.Cu") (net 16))
 (segment (start 145.861 -10.476) (end 145.861 9.714) (width 0.254) (layer "F.Cu") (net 16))
 (segment (start 145.861 9.714) (end 144.653 10.922) (width 0.254) (layer "F.Cu") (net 16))
 (segment (start 109.376 4.144) (end 110.438 5.207) (width 0.254) (layer "F.Cu") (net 11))
 (segment (start 110.438 5.207) (end 111.504 5.207) (width 0.254) (layer "F.Cu") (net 11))
 (segment (start 111.504 5.207) (end 119.761 13.464) (width 0.254) (layer "F.Cu") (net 11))
 (segment (start 119.761 13.464) (end 119.761 66.421) (width 0.254) (layer "F.Cu") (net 11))
 (segment (start 119.761 66.421) (end 125.603 72.263) (width 0.254) (layer "F.Cu") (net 11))
 (segment (start 103.505 -6.223) (end 105.918 -8.636) (width 0.254) (layer "F.Cu") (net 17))
 (segment (start 105.918 -8.636) (end 105.918 -12.987) (width 0.254) (layer "F.Cu") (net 17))
 (segment (start 105.918 -12.987) (end 106.482 -13.551) (width 0.254) (layer "F.Cu") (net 17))
 (segment (start 106.482 -13.551) (end 107.259 -13.551) (width 0.254) (layer "F.Cu") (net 17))
 (segment (start 107.259 -13.551) (end 129.54 8.73) (width 0.254) (layer "F.Cu") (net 17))
 (segment (start 129.54 8.73) (end 129.54 59.817) (width 0.254) (layer "F.Cu") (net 17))
 (segment (start 129.54 59.817) (end 134.038 64.315) (width 0.254) (layer "F.Cu") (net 17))
 (segment (start 134.038 64.315) (end 138.631 64.315) (width 0.254) (layer "F.Cu") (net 17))
 (segment (start 138.631 64.315) (end 139.827 63.119) (width 0.254) (layer "F.Cu") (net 17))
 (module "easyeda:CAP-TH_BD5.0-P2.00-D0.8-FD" (layer "F.Cu") (at 105.919 -12.573)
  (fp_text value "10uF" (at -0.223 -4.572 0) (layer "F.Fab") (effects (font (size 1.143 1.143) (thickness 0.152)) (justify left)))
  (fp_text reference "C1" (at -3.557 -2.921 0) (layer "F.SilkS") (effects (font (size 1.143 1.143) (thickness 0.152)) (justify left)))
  (pad 1 thru_hole circle (at -1 0 0) (size 1.3 1.3) (layers "*.Cu" "*.Paste" "*.Mask") (drill 0.8) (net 1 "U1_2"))
  (pad 2 thru_hole circle (at 1 0 0) (size 1.3 1.3) (layers "*.Cu" "*.Paste" "*.Mask") (drill 0.8) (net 10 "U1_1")))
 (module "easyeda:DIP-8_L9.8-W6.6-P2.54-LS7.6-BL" (layer "F.Cu") (at 148.59 -7.747 90)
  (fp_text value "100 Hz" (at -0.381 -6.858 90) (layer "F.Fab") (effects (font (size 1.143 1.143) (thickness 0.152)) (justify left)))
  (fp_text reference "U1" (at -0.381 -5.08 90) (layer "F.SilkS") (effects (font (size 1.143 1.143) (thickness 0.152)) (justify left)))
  (pad 1 thru_hole rect (at -3.81 3.81 90) (size 1.5 1.5) (layers "*.Cu" "*.Paste" "*.Mask") (drill 0.9) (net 10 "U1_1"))
  (pad 2 thru_hole circle (at -1.27 3.81 180) (size 1.5 1.5) (layers "*.Cu" "*.Paste" "*.Mask") (drill 0.9) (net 1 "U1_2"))
  (pad 3 thru_hole circle (at 1.27 3.81 180) (size 1.5 1.5) (layers "*.Cu" "*.Paste" "*.Mask") (drill 0.9) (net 8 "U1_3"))
  (pad 4 thru_hole circle (at 3.81 3.81 180) (size 1.5 1.5) (layers "*.Cu" "*.Paste" "*.Mask") (drill 0.9) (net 2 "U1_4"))
  (pad 8 thru_hole circle (at -3.81 -3.81 180) (size 1.5 1.5) (layers "*.Cu" "*.Paste" "*.Mask") (drill 0.9) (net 2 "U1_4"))
  (pad 7 thru_hole circle (at -1.27 -3.81 180) (size 1.5 1.5) (layers "*.Cu" "*.Paste" "*.Mask") (drill 0.9) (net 4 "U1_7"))
  (pad 6 thru_hole circle (at 1.27 -3.81 180) (size 1.5 1.5) (layers "*.Cu" "*.Paste" "*.Mask") (drill 0.9) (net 1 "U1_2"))
  (pad 5 thru_hole circle (at 3.81 -3.81 180) (size 1.5 1.5) (layers "*.Cu" "*.Paste" "*.Mask") (drill 0.9) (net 16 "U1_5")))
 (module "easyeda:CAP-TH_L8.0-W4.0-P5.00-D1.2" (layer "F.Cu") (at 142.113 10.922)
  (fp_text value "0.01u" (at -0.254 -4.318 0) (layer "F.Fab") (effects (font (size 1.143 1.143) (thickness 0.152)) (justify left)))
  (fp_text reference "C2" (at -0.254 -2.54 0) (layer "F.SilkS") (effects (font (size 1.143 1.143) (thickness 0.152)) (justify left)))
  (pad 1 thru_hole circle (at -2.54 0 0) (size 1.8 1.8) (layers "*.Cu" "*.Paste" "*.Mask") (drill 1.2) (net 10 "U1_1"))
  (pad 2 thru_hole circle (at 2.54 0 0) (size 1.8 1.8) (layers "*.Cu" "*.Paste" "*.Mask") (drill 1.2) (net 16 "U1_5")))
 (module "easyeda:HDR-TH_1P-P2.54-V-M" (layer "F.Cu") (at 114.935 12.065)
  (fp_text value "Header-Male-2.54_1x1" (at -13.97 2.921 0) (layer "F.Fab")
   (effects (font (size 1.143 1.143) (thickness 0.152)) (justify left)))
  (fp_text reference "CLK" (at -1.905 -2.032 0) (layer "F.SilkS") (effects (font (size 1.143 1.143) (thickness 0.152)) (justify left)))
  (pad 1 thru_hole rect (at 0 0 0) (size 1.7 1.7) (layers "*.Cu" "*.Paste" "*.Mask") (drill 1.1) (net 8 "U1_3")))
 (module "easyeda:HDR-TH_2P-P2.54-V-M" (layer "F.Cu") (at 151.638 4.191 90)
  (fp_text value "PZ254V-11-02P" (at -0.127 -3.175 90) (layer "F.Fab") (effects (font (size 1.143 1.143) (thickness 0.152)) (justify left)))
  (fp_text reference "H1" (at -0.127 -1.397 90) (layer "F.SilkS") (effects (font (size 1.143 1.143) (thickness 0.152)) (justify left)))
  (pad 1 thru_hole rect (at -1.27 0 90) (size 2 2) (layers "*.Cu" "*.Paste" "*.Mask") (drill 1.2) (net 2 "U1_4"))
  (pad 2 thru_hole circle (at 1.27 0 90) (size 2 2) (layers "*.Cu" "*.Paste" "*.Mask") (drill 1.2) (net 10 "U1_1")))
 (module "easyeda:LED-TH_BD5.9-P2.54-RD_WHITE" (layer "F.Cu") (at 124.587 25.019)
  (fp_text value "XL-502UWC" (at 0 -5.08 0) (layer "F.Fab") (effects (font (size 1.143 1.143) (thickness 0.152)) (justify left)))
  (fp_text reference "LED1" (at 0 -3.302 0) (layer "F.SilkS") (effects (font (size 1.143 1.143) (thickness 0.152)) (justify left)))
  (pad 1 thru_hole circle (at -1.27 0 0) (size 1.8 1.8) (layers "*.Cu" "*.Paste" "*.Mask") (drill 1) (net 9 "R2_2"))
  (pad 2 thru_hole circle (at 1.27 0 0) (size 1.8 1.8) (layers "*.Cu" "*.Paste" "*.Mask") (drill 1) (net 7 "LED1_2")))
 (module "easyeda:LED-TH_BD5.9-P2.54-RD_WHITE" (layer "F.Cu") (at 124.841 32.639)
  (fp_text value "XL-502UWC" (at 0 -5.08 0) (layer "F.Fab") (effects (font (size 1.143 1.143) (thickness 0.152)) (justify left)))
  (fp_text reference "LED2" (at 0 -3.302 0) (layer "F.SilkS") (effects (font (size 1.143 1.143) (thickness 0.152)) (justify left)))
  (pad 1 thru_hole circle (at -1.27 0 0) (size 1.8 1.8) (layers "*.Cu" "*.Paste" "*.Mask") (drill 1) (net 9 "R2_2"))
  (pad 2 thru_hole circle (at 1.27 0 0) (size 1.8 1.8) (layers "*.Cu" "*.Paste" "*.Mask") (drill 1) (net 6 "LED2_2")))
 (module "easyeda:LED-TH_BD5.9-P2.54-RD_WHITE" (layer "F.Cu") (at 125.095 40.259)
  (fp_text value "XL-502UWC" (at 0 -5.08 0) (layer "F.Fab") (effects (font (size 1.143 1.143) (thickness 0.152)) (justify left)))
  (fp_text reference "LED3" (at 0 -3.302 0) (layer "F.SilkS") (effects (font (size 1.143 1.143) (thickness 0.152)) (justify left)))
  (pad 1 thru_hole circle (at -1.27 0 0) (size 1.8 1.8) (layers "*.Cu" "*.Paste" "*.Mask") (drill 1) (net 9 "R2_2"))
  (pad 2 thru_hole circle (at 1.27 0 0) (size 1.8 1.8) (layers "*.Cu" "*.Paste" "*.Mask") (drill 1) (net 13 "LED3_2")))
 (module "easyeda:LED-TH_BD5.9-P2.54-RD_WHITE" (layer "F.Cu") (at 125.349 48.641)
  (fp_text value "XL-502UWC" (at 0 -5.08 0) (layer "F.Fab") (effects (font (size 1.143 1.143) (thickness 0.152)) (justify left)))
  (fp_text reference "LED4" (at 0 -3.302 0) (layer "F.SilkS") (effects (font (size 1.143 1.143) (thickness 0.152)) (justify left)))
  (pad 1 thru_hole circle (at -1.27 0 0) (size 1.8 1.8) (layers "*.Cu" "*.Paste" "*.Mask") (drill 1) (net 9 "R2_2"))
  (pad 2 thru_hole circle (at 1.27 0 0) (size 1.8 1.8) (layers "*.Cu" "*.Paste" "*.Mask") (drill 1) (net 15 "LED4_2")))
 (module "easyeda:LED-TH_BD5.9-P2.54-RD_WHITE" (layer "F.Cu") (at 124.841 57.023)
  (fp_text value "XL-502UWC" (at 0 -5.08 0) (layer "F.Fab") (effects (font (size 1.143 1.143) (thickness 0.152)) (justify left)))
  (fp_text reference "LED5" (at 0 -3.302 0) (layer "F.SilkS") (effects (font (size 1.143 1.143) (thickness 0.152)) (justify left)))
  (pad 1 thru_hole circle (at -1.27 0 0) (size 1.8 1.8) (layers "*.Cu" "*.Paste" "*.Mask") (drill 1) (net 9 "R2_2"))
  (pad 2 thru_hole circle (at 1.27 0 0) (size 1.8 1.8) (layers "*.Cu" "*.Paste" "*.Mask") (drill 1) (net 3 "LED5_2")))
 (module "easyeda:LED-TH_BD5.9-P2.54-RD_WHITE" (layer "F.Cu") (at 110.49 62.992)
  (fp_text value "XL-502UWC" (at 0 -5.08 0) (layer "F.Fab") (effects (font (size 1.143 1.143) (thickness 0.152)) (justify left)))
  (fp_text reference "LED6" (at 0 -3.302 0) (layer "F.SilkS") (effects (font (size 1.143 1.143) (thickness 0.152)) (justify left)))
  (pad 1 thru_hole circle (at -1.27 0 0) (size 1.8 1.8) (layers "*.Cu" "*.Paste" "*.Mask") (drill 1) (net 9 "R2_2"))
  (pad 2 thru_hole circle (at 1.27 0 0) (size 1.8 1.8) (layers "*.Cu" "*.Paste" "*.Mask") (drill 1) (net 12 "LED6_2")))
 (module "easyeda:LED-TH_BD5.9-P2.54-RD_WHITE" (layer "F.Cu") (at 119.761 65.024)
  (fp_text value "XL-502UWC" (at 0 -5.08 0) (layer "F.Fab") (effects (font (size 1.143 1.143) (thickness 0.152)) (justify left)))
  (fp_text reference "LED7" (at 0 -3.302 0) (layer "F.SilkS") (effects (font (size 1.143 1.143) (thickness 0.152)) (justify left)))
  (pad 1 thru_hole circle (at -1.27 0 0) (size 1.8 1.8) (layers "*.Cu" "*.Paste" "*.Mask") (drill 1) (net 9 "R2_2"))
  (pad 2 thru_hole circle (at 1.27 0 0) (size 1.8 1.8) (layers "*.Cu" "*.Paste" "*.Mask") (drill 1) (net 14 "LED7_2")))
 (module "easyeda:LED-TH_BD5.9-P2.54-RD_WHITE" (layer "F.Cu") (at 129.286 65.151)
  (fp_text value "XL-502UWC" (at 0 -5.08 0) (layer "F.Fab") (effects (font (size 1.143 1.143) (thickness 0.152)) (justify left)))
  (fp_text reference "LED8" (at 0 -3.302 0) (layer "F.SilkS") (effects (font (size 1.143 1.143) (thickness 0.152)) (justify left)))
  (pad 1 thru_hole circle (at -1.27 0 0) (size 1.8 1.8) (layers "*.Cu" "*.Paste" "*.Mask") (drill 1) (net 9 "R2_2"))
  (pad 2 thru_hole circle (at 1.27 0 0) (size 1.8 1.8) (layers "*.Cu" "*.Paste" "*.Mask") (drill 1) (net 5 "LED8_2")))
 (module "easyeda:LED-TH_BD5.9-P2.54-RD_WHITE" (layer "F.Cu") (at 138.557 63.119)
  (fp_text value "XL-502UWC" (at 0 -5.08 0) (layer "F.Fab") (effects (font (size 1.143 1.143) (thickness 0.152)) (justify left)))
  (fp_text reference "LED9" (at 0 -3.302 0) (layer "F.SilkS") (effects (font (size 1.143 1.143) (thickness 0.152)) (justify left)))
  (pad 1 thru_hole circle (at -1.27 0 0) (size 1.8 1.8) (layers "*.Cu" "*.Paste" "*.Mask") (drill 1) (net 9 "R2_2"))
  (pad 2 thru_hole circle (at 1.27 0 0) (size 1.8 1.8) (layers "*.Cu" "*.Paste" "*.Mask") (drill 1) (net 17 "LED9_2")))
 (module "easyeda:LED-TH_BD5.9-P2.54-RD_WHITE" (layer "F.Cu") (at 124.333 72.263)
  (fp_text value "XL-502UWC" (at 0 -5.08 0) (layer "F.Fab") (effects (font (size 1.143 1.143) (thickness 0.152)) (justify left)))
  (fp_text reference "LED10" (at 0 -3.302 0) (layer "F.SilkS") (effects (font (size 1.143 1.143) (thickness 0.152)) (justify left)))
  (pad 1 thru_hole circle (at -1.27 0 0) (size 1.8 1.8) (layers "*.Cu" "*.Paste" "*.Mask") (drill 1) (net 9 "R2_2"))
  (pad 2 thru_hole circle (at 1.27 0 0) (size 1.8 1.8) (layers "*.Cu" "*.Paste" "*.Mask") (drill 1) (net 11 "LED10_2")))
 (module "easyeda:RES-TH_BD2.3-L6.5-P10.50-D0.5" (layer "F.Cu") (at 133.35 -12.827)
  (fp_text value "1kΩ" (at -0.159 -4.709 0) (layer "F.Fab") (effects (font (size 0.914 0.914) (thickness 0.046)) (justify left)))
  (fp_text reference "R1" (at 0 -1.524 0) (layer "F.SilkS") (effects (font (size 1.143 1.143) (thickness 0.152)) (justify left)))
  (pad 1 thru_hole circle (at -5.25 0 0) (size 1.4 1.4) (layers "*.Cu" "*.Paste" "*.Mask") (drill 0.7) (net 4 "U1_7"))
  (pad 2 thru_hole circle (at 5.25 0 0) (size 1.4 1.4) (layers "*.Cu" "*.Paste" "*.Mask") (drill 0.7) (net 2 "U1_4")))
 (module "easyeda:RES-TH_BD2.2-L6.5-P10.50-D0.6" (layer "F.Cu") (at 97.155 -0.381 90)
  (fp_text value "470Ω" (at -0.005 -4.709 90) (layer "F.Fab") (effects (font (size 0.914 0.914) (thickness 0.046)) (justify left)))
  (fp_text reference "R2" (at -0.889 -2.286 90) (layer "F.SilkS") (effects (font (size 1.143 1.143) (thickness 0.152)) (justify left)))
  (pad 1 thru_hole circle (at -5.25 0 90) (size 1.6 1.6) (layers "*.Cu" "*.Paste" "*.Mask") (drill 0.914) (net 10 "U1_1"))
  (pad 2 thru_hole circle (at 5.25 0 90) (size 1.6 1.6) (layers "*.Cu" "*.Paste" "*.Mask") (drill 0.914) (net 9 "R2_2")))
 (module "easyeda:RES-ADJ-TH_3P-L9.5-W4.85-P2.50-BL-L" (layer "F.Cu") (at 118.364 -11.811 90)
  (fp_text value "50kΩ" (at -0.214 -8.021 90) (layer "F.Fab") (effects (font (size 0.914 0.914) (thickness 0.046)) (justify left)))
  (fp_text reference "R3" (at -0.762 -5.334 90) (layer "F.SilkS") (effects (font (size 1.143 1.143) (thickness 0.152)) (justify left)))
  (pad 2 thru_hole circle (at 0 0 0) (size 1.524 1.524) (layers "*.Cu" "*.Paste" "*.Mask") (drill 0.762) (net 4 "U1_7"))
  (pad 1 thru_hole circle (at 0 -2.5 0) (size 1.524 1.524) (layers "*.Cu" "*.Paste" "*.Mask") (drill 0.762) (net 1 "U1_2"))
  (pad 3 thru_hole circle (at 0 2.5 0) (size 1.524 1.524) (layers "*.Cu" "*.Paste" "*.Mask") (drill 0.762) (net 4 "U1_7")))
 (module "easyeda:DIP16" (layer "F.Cu") (at 107.315 2.667 90)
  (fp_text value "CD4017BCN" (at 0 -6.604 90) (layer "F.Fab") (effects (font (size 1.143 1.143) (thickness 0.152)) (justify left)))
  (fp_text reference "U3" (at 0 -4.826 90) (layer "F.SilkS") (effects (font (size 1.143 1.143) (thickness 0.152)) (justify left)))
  (pad 1 thru_hole rect (at -8.89 3.81 90) (size 1.397 1.397) (layers "*.Cu" "*.Paste" "*.Mask") (drill 0.711) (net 12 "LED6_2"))
  (pad 2 thru_hole circle (at -6.35 3.81 90) (size 1.397 1.397) (layers "*.Cu" "*.Paste" "*.Mask") (drill 0.711) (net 6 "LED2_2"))
  (pad 3 thru_hole circle (at -3.81 3.81 90) (size 1.397 1.397) (layers "*.Cu" "*.Paste" "*.Mask") (drill 0.711) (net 7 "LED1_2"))
  (pad 4 thru_hole circle (at -1.27 3.81 90) (size 1.397 1.397) (layers "*.Cu" "*.Paste" "*.Mask") (drill 0.711) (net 13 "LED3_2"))
  (pad 5 thru_hole circle (at 1.27 3.81 90) (size 1.397 1.397) (layers "*.Cu" "*.Paste" "*.Mask") (drill 0.711) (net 14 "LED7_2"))
  (pad 6 thru_hole circle (at 3.81 3.81 90) (size 1.397 1.397) (layers "*.Cu" "*.Paste" "*.Mask") (drill 0.711) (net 5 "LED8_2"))
  (pad 7 thru_hole circle (at 6.35 3.81 90) (size 1.397 1.397) (layers "*.Cu" "*.Paste" "*.Mask") (drill 0.711) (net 15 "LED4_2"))
  (pad 8 thru_hole circle (at 8.89 3.81 90) (size 1.397 1.397) (layers "*.Cu" "*.Paste" "*.Mask") (drill 0.711) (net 10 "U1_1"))
  (pad 9 thru_hole circle (at 8.89 -3.81 90) (size 1.397 1.397) (layers "*.Cu" "*.Paste" "*.Mask") (drill 0.711) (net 17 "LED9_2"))
  (pad 10 thru_hole circle (at 6.35 -3.81 90) (size 1.397 1.397) (layers "*.Cu" "*.Paste" "*.Mask") (drill 0.711) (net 3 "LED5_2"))
  (pad 11 thru_hole circle (at 3.81 -3.81 90) (size 1.397 1.397) (layers "*.Cu" "*.Paste" "*.Mask") (drill 0.711) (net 11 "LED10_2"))
  (pad 12 thru_hole circle (at 1.27 -3.81 90) (size 1.397 1.397) (layers "*.Cu" "*.Paste" "*.Mask") (drill 0.711))
  (pad 13 thru_hole circle (at -1.27 -3.81 90) (size 1.397 1.397) (layers "*.Cu" "*.Paste" "*.Mask") (drill 0.711) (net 10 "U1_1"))
  (pad 14 thru_hole circle (at -3.81 -3.81 90) (size 1.397 1.397) (layers "*.Cu" "*.Paste" "*.Mask") (drill 0.711) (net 8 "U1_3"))
  (pad 15 thru_hole circle (at -6.35 -3.81 90) (size 1.397 1.397) (layers "*.Cu" "*.Paste" "*.Mask") (drill 0.711) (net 10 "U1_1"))
  (pad 16 thru_hole circle (at -8.89 -3.81 90) (size 1.397 1.397) (layers "*.Cu" "*.Paste" "*.Mask") (drill 0.711) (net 2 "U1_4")))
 (via (at 127.804 11.181) (size 0.61) (drill 0.305) (layers "F.Cu" "B.Cu") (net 3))
 (via (at 118.588 57.102) (size 0.61) (drill 0.305) (layers "F.Cu" "B.Cu") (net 12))
 (via (at 109.375 4.144) (size 0.61) (drill 0.305) (layers "F.Cu" "B.Cu") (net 11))
 (via (at 122.025 11.284) (size 0.61) (drill 0.305) (layers "F.Cu" "B.Cu") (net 5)))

